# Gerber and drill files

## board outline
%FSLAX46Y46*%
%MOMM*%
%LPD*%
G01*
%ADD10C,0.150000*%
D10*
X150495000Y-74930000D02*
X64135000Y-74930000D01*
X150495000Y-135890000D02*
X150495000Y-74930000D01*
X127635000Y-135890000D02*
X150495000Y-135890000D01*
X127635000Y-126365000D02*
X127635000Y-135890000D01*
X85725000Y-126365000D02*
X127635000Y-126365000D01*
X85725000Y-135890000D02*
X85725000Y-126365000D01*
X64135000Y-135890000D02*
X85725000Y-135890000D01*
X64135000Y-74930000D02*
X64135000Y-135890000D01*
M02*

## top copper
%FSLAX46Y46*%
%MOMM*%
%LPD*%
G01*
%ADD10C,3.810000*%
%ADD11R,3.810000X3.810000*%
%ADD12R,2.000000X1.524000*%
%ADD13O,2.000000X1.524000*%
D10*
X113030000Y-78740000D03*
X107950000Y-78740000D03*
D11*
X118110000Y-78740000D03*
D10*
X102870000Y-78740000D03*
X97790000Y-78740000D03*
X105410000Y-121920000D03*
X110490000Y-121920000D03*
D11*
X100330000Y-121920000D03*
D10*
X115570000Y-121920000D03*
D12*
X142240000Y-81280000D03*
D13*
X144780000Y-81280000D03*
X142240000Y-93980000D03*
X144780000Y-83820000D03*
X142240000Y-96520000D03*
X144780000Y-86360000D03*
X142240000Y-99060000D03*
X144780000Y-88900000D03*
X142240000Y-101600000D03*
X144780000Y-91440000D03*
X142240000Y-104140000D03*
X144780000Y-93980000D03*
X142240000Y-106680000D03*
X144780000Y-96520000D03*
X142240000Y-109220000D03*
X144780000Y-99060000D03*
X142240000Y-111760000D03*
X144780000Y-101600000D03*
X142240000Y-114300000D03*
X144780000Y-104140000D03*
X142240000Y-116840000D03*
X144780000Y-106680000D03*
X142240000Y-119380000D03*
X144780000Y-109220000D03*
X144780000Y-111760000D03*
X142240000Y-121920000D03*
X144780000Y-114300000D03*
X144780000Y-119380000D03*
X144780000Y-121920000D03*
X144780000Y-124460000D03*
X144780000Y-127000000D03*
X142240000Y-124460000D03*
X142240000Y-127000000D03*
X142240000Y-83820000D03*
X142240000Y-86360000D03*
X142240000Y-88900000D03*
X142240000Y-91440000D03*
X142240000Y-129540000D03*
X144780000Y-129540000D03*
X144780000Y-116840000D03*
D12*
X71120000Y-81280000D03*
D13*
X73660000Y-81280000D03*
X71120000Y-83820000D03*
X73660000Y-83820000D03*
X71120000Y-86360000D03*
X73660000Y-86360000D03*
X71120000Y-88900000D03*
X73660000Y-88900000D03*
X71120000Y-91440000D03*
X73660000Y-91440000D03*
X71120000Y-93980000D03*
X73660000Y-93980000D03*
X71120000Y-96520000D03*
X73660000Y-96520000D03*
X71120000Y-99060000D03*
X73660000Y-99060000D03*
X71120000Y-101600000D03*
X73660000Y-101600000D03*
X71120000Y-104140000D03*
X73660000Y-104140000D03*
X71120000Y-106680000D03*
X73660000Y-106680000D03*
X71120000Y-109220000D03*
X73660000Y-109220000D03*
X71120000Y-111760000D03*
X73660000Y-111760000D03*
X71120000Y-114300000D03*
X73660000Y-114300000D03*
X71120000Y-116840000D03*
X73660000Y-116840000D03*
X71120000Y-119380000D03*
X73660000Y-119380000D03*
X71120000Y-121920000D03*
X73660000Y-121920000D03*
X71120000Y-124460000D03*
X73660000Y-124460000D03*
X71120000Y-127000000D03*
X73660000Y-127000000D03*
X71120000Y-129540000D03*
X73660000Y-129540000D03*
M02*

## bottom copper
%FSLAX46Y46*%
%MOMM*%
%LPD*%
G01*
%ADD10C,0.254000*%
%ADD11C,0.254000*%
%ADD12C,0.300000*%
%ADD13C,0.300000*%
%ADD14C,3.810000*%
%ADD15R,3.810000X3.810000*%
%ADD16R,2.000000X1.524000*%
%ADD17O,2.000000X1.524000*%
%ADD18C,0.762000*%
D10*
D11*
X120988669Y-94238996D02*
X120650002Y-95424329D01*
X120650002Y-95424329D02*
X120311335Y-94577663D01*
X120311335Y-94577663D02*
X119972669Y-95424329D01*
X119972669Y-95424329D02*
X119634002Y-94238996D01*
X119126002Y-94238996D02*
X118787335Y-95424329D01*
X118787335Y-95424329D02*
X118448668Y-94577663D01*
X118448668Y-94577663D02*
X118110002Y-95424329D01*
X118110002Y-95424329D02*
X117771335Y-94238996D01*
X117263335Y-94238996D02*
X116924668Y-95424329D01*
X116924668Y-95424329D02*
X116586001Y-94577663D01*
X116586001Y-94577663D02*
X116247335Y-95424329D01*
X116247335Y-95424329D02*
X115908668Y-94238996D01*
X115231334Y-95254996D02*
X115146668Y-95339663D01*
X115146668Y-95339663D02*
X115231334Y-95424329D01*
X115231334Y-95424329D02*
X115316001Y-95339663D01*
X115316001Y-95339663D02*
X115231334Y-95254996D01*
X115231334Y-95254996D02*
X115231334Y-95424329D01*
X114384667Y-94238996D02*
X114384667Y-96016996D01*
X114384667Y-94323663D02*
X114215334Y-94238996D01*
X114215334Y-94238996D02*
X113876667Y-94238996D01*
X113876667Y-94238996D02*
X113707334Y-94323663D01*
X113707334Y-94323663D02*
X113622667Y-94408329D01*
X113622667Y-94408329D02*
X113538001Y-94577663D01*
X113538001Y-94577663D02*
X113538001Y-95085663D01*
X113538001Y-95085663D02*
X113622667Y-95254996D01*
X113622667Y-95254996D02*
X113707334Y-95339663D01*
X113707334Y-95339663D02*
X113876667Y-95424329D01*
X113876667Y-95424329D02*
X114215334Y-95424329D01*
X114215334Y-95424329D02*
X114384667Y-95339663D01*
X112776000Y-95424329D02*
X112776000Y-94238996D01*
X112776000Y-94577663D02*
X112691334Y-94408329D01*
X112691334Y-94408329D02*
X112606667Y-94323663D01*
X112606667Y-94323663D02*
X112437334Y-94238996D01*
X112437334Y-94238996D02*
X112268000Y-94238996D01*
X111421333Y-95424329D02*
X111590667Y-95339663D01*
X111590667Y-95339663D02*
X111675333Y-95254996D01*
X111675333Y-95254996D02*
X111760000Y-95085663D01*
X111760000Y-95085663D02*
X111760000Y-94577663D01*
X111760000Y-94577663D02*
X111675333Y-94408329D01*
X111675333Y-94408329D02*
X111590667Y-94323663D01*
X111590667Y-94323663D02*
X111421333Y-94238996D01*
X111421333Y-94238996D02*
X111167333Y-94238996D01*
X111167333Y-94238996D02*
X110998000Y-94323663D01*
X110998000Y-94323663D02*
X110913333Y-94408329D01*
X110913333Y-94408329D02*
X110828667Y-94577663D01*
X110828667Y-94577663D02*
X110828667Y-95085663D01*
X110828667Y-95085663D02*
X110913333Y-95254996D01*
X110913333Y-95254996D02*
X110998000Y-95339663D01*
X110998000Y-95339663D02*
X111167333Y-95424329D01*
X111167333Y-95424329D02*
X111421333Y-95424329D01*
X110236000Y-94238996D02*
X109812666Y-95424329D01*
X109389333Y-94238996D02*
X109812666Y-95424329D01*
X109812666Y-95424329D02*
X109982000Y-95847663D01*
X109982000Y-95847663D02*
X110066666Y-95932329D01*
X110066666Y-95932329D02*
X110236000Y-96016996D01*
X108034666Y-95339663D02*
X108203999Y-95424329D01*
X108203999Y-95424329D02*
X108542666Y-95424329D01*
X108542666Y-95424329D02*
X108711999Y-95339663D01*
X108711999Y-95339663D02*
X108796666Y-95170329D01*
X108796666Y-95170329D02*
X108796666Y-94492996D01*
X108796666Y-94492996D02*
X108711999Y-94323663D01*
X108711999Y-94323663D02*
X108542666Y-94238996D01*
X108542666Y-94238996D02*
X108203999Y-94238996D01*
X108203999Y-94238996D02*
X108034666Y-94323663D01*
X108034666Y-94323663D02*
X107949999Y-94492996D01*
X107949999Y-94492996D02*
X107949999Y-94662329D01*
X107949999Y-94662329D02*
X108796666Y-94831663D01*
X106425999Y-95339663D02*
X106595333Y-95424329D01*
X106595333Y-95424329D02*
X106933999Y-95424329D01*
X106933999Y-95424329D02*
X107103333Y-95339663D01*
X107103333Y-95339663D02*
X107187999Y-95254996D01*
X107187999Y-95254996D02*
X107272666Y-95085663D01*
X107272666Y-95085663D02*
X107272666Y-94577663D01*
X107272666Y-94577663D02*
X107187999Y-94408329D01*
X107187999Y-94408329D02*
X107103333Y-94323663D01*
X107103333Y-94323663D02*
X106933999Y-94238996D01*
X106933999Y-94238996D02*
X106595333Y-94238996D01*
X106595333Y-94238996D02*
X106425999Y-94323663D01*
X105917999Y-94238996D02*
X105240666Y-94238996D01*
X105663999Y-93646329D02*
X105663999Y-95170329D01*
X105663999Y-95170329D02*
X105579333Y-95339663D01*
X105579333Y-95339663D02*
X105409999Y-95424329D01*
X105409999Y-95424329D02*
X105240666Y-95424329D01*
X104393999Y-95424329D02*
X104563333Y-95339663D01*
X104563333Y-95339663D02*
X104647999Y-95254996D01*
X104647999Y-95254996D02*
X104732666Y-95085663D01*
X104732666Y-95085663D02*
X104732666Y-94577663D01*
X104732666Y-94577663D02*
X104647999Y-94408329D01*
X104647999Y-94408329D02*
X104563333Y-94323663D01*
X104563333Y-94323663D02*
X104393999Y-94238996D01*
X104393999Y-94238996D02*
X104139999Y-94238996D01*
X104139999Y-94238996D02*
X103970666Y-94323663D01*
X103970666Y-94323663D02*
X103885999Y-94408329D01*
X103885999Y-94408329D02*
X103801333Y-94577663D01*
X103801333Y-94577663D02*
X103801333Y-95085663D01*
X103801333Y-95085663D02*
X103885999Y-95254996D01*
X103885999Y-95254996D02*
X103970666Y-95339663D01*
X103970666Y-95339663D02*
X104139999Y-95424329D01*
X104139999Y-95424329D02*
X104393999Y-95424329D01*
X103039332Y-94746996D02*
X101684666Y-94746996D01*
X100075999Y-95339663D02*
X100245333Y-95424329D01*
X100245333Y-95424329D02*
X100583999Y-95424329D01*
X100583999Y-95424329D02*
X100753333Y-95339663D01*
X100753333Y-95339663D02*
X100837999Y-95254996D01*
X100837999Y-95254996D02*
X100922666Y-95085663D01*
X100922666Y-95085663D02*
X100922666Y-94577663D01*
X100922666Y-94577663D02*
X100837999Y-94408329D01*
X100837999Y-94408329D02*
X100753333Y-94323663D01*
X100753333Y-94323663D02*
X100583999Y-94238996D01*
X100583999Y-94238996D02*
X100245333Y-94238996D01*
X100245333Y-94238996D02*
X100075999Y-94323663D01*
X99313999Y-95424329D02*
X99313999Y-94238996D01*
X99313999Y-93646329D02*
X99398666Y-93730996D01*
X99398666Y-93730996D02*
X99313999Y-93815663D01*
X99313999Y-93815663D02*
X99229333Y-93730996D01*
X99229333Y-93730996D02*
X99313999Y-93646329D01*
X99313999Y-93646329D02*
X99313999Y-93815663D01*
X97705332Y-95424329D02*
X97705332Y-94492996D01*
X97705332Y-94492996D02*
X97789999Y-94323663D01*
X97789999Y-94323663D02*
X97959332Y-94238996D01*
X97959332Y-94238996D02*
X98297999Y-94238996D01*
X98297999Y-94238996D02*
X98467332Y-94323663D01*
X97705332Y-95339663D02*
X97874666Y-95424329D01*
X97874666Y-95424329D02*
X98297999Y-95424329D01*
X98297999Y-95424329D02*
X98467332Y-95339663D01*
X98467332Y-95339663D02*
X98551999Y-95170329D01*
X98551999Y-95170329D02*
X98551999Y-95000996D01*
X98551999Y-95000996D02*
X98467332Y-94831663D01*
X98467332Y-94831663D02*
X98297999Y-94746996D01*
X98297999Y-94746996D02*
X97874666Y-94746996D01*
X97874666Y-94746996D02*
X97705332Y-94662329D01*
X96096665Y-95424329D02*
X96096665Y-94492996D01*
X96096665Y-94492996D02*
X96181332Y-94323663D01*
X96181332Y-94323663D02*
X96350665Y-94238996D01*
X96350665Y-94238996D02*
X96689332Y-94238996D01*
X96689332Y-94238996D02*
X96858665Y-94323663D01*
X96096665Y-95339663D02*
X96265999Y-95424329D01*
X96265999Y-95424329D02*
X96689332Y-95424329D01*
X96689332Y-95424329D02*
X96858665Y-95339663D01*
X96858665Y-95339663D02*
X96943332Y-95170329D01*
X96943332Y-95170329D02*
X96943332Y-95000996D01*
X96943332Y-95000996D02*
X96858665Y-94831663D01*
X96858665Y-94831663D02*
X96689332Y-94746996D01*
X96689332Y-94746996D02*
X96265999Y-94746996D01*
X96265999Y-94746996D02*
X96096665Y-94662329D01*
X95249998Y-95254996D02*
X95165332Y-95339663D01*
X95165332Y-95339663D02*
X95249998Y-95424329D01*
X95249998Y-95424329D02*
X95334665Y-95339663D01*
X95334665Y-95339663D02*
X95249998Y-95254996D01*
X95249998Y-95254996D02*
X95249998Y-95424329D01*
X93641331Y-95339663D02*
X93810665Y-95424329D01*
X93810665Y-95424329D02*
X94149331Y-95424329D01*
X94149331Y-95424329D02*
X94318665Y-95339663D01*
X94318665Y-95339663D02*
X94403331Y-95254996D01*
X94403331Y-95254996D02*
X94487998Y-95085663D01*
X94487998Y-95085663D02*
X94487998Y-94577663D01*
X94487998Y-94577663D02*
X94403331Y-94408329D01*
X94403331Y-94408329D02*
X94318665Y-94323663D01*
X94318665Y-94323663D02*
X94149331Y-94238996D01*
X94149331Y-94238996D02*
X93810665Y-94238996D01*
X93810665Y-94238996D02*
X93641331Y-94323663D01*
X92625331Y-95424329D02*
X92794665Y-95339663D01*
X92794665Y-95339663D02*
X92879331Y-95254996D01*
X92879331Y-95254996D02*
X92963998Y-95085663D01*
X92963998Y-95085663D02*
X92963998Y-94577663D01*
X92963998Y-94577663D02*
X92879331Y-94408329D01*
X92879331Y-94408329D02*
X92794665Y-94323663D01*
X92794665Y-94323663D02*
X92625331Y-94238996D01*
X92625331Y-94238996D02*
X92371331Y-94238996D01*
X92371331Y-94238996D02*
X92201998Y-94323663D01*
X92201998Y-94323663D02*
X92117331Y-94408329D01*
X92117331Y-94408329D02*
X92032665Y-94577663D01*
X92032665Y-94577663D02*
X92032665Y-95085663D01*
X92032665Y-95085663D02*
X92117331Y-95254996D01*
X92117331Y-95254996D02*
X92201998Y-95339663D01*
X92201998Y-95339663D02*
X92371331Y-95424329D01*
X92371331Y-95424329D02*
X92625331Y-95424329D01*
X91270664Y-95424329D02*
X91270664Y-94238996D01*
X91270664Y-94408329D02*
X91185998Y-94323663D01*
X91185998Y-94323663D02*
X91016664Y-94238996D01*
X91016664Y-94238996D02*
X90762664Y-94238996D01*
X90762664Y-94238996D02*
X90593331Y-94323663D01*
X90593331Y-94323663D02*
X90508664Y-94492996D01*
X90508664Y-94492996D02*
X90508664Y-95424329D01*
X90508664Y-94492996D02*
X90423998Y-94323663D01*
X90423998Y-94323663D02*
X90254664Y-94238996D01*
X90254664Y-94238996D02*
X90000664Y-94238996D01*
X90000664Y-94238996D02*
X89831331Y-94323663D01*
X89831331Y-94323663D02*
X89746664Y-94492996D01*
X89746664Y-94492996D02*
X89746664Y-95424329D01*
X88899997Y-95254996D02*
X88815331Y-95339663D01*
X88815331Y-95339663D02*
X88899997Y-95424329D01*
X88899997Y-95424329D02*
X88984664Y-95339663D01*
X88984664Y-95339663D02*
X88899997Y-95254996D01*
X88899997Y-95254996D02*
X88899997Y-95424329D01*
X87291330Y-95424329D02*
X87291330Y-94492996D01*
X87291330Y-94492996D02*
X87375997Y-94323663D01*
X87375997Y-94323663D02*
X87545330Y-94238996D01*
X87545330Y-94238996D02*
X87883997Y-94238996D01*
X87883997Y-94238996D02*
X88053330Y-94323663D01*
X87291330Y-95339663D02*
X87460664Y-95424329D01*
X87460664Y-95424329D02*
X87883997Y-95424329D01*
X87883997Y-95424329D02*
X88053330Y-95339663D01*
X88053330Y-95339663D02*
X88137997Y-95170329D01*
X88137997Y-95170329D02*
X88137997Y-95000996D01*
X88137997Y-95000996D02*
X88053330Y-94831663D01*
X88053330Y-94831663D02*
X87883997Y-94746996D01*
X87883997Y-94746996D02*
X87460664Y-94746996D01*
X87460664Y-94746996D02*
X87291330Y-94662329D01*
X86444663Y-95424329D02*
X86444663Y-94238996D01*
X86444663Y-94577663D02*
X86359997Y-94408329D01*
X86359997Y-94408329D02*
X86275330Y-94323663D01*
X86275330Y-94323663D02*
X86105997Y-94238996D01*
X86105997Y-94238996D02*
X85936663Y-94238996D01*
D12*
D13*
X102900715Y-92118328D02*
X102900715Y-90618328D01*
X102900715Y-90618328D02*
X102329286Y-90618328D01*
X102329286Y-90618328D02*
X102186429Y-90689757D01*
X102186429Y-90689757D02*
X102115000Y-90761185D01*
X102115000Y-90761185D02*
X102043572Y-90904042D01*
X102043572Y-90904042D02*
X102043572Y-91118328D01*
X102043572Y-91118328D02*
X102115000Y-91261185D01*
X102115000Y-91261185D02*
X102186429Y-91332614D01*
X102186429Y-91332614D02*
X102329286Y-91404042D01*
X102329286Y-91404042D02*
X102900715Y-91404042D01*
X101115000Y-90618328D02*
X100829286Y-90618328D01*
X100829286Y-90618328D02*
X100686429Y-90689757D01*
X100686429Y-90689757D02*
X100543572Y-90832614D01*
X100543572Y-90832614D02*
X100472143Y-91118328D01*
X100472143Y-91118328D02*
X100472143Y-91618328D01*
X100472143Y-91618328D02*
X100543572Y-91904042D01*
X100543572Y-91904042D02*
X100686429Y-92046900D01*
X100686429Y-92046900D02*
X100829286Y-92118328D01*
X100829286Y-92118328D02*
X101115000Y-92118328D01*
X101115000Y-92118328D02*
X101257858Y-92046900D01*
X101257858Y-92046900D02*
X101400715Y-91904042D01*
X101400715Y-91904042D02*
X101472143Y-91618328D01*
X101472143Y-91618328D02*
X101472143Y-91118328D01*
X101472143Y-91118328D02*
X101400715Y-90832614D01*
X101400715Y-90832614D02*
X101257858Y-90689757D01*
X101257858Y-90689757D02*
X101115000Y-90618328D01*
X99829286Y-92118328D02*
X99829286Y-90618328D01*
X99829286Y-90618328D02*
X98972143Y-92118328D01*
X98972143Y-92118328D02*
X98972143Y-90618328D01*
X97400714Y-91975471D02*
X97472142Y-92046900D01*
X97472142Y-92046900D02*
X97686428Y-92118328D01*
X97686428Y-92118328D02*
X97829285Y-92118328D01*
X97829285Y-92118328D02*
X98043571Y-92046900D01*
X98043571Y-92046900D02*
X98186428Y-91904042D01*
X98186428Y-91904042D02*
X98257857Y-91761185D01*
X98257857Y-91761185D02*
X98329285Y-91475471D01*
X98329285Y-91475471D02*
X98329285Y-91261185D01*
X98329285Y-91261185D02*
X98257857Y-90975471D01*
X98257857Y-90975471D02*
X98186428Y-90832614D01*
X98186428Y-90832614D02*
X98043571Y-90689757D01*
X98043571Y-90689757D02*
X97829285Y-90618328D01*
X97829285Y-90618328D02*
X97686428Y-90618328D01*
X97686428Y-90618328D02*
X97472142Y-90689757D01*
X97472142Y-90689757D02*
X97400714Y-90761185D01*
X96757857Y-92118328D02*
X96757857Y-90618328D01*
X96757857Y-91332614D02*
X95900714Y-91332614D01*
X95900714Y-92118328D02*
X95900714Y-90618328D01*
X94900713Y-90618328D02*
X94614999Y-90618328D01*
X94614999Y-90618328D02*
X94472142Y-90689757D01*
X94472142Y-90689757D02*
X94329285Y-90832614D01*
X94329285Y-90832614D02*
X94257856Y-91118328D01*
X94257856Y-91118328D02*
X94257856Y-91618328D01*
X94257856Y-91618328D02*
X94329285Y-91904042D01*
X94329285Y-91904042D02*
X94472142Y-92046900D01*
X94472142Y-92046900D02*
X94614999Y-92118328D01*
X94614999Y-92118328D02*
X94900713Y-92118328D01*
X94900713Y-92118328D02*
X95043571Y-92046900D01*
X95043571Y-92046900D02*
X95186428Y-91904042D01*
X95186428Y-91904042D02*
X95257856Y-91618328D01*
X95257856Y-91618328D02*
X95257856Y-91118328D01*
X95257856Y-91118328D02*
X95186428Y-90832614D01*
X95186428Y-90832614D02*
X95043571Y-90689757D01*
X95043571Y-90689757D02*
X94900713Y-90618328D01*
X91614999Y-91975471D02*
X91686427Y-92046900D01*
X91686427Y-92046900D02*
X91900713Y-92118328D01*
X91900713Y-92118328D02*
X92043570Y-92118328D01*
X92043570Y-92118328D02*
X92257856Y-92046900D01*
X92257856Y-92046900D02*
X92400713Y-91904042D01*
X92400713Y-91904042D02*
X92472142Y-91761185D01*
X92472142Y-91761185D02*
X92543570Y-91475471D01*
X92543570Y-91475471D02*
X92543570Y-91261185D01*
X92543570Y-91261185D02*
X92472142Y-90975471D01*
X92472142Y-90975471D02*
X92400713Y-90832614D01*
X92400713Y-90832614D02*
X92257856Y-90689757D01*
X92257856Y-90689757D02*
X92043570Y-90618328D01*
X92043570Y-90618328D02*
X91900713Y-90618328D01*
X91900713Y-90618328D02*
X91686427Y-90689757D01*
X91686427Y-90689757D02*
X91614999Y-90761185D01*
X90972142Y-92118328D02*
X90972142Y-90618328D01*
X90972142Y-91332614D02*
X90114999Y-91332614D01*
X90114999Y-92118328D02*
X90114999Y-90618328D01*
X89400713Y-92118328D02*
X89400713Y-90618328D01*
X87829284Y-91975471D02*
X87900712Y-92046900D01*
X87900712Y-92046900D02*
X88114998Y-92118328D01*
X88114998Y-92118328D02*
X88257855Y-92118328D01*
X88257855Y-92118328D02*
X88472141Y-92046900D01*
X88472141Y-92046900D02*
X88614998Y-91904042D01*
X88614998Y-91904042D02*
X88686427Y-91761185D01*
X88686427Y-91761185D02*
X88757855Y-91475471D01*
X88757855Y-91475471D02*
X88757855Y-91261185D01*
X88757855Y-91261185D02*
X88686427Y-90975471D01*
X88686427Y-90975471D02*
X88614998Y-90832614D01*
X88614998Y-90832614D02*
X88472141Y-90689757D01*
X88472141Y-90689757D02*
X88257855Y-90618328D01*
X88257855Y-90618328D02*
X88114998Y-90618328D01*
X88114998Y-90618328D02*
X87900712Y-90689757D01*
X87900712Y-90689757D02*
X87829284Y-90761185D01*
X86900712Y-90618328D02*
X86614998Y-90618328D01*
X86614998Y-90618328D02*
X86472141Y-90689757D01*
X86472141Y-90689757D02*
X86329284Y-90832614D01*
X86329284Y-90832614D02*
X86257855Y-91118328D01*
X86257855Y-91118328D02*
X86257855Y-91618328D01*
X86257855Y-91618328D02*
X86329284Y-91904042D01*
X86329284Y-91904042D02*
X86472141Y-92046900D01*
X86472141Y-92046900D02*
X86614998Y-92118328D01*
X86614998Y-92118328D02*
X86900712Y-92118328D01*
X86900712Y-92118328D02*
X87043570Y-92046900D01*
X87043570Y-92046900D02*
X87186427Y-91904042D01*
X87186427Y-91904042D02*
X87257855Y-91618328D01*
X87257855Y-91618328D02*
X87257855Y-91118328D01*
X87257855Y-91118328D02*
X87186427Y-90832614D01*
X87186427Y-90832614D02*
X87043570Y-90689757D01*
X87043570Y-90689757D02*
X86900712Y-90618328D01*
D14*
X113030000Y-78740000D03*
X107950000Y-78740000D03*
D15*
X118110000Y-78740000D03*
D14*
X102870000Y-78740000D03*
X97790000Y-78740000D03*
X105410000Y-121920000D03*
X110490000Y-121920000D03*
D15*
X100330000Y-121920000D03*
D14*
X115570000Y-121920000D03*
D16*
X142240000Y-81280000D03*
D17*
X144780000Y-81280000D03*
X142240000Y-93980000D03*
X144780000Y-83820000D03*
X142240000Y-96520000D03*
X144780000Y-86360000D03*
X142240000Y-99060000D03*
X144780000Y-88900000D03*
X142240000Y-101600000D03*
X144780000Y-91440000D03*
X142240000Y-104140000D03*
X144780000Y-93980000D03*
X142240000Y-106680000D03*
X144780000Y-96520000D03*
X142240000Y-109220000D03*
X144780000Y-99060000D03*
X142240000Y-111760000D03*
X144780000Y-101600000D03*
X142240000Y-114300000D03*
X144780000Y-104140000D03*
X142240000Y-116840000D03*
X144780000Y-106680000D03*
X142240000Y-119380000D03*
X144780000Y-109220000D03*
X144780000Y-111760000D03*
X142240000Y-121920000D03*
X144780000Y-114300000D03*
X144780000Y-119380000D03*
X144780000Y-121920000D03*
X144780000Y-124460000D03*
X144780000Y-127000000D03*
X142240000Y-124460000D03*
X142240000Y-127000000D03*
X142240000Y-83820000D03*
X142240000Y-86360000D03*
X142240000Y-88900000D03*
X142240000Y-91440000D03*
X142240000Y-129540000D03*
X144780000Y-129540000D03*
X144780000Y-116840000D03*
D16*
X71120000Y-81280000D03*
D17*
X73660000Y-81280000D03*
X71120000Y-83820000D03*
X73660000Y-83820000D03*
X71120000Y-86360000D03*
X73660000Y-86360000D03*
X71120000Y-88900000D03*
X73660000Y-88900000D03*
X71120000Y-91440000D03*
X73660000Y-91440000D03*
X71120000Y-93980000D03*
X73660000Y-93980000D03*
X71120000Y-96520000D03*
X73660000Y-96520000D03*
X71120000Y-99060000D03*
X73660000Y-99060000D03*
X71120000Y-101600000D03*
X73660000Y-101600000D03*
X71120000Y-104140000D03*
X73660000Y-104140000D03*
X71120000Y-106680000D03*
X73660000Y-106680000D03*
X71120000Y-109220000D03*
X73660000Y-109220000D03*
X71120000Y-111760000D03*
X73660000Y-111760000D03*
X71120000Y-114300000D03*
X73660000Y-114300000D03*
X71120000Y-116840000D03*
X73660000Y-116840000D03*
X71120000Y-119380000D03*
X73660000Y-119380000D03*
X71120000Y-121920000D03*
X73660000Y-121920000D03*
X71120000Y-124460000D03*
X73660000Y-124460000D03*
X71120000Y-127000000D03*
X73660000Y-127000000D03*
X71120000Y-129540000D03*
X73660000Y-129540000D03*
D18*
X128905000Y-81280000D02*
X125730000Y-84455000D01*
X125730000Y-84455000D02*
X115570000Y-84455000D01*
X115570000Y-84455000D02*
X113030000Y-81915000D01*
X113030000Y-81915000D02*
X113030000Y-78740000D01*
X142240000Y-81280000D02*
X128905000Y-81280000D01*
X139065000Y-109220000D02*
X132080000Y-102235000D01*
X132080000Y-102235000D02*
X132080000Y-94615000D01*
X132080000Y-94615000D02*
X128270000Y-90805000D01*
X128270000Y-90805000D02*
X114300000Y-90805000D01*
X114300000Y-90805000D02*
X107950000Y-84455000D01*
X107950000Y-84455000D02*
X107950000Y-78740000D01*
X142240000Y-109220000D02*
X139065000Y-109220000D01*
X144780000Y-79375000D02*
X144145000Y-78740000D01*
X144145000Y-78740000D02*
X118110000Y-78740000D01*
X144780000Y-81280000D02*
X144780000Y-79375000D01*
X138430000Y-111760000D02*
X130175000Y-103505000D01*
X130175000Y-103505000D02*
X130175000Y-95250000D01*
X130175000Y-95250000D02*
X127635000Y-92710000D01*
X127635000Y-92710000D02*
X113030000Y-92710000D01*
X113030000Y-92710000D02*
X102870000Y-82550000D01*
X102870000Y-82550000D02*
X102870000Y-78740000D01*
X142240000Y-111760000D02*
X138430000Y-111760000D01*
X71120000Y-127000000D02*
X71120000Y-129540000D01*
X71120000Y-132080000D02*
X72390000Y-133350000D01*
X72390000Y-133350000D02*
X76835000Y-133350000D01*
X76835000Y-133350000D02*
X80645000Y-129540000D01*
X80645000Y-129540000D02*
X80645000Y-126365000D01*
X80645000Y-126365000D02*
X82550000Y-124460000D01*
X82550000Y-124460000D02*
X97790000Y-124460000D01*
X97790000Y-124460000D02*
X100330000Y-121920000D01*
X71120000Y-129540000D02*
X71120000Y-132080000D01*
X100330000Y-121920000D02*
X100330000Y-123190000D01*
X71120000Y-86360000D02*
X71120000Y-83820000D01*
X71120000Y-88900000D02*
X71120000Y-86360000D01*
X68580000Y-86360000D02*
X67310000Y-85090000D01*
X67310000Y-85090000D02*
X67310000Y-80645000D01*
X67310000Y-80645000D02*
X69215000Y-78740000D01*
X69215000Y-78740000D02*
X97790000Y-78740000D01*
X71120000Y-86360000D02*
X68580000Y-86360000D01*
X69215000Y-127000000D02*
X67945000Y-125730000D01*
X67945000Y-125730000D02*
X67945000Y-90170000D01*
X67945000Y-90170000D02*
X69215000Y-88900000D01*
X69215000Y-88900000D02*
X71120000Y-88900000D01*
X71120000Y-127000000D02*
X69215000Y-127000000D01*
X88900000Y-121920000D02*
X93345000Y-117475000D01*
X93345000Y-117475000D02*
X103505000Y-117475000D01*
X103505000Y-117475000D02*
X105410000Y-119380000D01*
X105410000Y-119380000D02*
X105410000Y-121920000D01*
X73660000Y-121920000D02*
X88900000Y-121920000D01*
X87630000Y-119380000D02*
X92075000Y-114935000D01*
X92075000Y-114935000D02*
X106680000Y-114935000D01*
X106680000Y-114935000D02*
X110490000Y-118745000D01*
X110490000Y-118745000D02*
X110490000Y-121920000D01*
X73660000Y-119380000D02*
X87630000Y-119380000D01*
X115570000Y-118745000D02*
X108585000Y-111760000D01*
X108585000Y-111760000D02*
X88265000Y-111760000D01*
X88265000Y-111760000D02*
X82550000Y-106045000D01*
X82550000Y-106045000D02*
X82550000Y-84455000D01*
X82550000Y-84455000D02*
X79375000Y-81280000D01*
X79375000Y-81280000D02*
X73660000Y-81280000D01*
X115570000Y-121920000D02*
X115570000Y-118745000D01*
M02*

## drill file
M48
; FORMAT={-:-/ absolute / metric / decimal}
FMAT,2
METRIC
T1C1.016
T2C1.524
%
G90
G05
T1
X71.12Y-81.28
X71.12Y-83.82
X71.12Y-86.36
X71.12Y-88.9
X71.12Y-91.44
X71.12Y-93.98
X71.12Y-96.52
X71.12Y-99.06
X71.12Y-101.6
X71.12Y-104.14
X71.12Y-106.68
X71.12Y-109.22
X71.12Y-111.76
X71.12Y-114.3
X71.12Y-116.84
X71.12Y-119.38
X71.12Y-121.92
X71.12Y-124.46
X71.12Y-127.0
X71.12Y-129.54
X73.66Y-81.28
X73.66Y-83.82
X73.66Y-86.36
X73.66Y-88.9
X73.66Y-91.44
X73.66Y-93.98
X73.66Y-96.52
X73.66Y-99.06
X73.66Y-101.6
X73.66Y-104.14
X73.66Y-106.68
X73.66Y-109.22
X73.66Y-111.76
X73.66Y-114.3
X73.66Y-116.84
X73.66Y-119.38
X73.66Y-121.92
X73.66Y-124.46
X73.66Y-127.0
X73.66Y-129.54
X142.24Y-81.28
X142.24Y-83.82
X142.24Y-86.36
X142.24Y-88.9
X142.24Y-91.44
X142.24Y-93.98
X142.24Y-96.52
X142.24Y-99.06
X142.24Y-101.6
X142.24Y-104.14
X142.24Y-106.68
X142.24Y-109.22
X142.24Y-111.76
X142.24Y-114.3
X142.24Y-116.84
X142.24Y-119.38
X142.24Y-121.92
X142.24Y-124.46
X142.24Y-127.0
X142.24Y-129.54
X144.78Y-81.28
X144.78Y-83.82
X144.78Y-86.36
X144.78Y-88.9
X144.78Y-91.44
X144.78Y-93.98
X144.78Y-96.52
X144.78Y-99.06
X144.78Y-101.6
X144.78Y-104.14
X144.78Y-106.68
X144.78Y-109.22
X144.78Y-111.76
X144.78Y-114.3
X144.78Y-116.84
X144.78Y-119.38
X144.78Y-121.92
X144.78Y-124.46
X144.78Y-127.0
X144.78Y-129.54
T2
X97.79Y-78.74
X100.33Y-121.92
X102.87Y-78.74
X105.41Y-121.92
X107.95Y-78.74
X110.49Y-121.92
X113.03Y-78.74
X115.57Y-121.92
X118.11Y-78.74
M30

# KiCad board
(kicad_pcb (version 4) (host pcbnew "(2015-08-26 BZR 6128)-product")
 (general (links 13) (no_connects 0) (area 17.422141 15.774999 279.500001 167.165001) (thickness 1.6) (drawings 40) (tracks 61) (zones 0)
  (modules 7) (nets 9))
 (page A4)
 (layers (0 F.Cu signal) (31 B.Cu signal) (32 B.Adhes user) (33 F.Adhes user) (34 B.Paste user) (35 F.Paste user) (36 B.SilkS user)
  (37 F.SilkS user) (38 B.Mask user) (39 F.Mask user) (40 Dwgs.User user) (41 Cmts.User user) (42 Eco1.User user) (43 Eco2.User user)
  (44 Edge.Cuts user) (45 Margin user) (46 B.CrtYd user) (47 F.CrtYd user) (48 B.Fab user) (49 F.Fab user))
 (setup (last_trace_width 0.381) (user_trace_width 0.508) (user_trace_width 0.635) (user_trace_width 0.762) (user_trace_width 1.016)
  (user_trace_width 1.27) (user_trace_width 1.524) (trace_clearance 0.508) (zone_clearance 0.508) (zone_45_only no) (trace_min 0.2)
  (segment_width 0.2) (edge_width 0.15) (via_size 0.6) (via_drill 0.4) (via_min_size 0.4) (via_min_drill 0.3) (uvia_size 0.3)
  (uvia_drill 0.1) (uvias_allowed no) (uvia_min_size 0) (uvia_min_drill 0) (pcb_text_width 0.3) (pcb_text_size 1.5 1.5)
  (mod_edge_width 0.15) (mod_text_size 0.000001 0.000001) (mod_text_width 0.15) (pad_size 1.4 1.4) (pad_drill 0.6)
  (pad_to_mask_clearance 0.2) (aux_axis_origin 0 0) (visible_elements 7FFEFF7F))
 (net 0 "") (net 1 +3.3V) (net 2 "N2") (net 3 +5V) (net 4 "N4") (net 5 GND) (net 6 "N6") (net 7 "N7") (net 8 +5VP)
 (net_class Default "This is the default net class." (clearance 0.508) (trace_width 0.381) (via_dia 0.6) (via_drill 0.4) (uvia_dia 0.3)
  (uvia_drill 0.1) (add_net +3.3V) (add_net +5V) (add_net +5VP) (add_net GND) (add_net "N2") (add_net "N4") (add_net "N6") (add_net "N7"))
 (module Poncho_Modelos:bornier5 (layer F.Cu) (at 107.95 78.74 180)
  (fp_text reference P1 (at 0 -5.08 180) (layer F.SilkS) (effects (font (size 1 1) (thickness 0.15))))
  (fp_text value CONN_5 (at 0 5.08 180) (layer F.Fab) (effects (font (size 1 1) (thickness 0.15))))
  (pad 2 thru_hole circle (at -5.08 0 180) (size 3.81 3.81) (drill 1.524) (layers *.Cu *.Mask F.SilkS) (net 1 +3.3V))
  (pad 3 thru_hole circle (at 0 0 180) (size 3.81 3.81) (drill 1.524) (layers *.Cu *.Mask F.SilkS) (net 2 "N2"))
  (pad 1 thru_hole rect (at -10.16 0 180) (size 3.81 3.81) (drill 1.524) (layers *.Cu *.Mask F.SilkS) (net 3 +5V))
  (pad 4 thru_hole circle (at 5.08 0 180) (size 3.81 3.81) (drill 1.524) (layers *.Cu *.Mask F.SilkS) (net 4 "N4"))
  (pad 5 thru_hole circle (at 10.16 0 180) (size 3.81 3.81) (drill 1.524) (layers *.Cu *.Mask F.SilkS) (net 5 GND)))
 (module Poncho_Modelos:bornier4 (layer F.Cu) (at 107.95 121.92)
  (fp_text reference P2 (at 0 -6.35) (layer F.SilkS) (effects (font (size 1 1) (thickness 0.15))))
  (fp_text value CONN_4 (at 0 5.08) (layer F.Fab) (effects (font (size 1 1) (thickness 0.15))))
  (pad 2 thru_hole circle (at -2.54 0) (size 3.81 3.81) (drill 1.524) (layers *.Cu *.Mask F.SilkS) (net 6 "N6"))
  (pad 3 thru_hole circle (at 2.54 0) (size 3.81 3.81) (drill 1.524) (layers *.Cu *.Mask F.SilkS) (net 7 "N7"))
  (pad 1 thru_hole rect (at -7.62 0) (size 3.81 3.81) (drill 1.524) (layers *.Cu *.Mask F.SilkS) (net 5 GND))
  (pad 4 thru_hole circle (at 7.62 0) (size 3.81 3.81) (drill 1.524) (layers *.Cu *.Mask F.SilkS) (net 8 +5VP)))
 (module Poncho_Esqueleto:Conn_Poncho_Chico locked (layer F.Cu) (at 142.24 81.28)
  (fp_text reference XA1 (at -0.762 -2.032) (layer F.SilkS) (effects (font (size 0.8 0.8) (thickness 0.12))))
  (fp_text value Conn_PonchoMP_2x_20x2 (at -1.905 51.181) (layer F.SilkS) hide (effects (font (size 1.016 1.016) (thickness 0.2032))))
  (pad 1 thru_hole rect (at 0 0 270) (size 1.524 2) (drill 1.016) (layers *.Cu *.Mask F.SilkS) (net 1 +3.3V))
  (pad 2 thru_hole oval (at 2.54 0 270) (size 1.524 2) (drill 1.016) (layers *.Cu *.Mask F.SilkS) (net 3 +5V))
  (pad 11 thru_hole oval (at 0 12.7 270) (size 1.524 2) (drill 1.016) (layers *.Cu *.Mask F.SilkS))
  (pad 4 thru_hole oval (at 2.54 2.54 270) (size 1.524 2) (drill 1.016) (layers *.Cu *.Mask F.SilkS))
  (pad 13 thru_hole oval (at 0 15.24 270) (size 1.524 2) (drill 1.016) (layers *.Cu *.Mask F.SilkS))
  (pad 6 thru_hole oval (at 2.54 5.08 270) (size 1.524 2) (drill 1.016) (layers *.Cu *.Mask F.SilkS))
  (pad 15 thru_hole oval (at 0 17.78 270) (size 1.524 2) (drill 1.016) (layers *.Cu *.Mask F.SilkS))
  (pad 8 thru_hole oval (at 2.54 7.62 270) (size 1.524 2) (drill 1.016) (layers *.Cu *.Mask F.SilkS))
  (pad 17 thru_hole oval (at 0 20.32 270) (size 1.524 2) (drill 1.016) (layers *.Cu *.Mask F.SilkS))
  (pad 10 thru_hole oval (at 2.54 10.16 270) (size 1.524 2) (drill 1.016) (layers *.Cu *.Mask F.SilkS))
  (pad 19 thru_hole oval (at 0 22.86 270) (size 1.524 2) (drill 1.016) (layers *.Cu *.Mask F.SilkS))
  (pad 12 thru_hole oval (at 2.54 12.7 270) (size 1.524 2) (drill 1.016) (layers *.Cu *.Mask F.SilkS))
  (pad 21 thru_hole oval (at 0 25.4 270) (size 1.524 2) (drill 1.016) (layers *.Cu *.Mask F.SilkS))
  (pad 14 thru_hole oval (at 2.54 15.24 270) (size 1.524 2) (drill 1.016) (layers *.Cu *.Mask F.SilkS))
  (pad 23 thru_hole oval (at 0 27.94 270) (size 1.524 2) (drill 1.016) (layers *.Cu *.Mask F.SilkS) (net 2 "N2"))
  (pad 16 thru_hole oval (at 2.54 17.78 270) (size 1.524 2) (drill 1.016) (layers *.Cu *.Mask F.SilkS))
  (pad 25 thru_hole oval (at 0 30.48 270) (size 1.524 2) (drill 1.016) (layers *.Cu *.Mask F.SilkS) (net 4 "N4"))
  (pad 18 thru_hole oval (at 2.54 20.32 270) (size 1.524 2) (drill 1.016) (layers *.Cu *.Mask F.SilkS))
  (pad 27 thru_hole oval (at 0 33.02 270) (size 1.524 2) (drill 1.016) (layers *.Cu *.Mask F.SilkS))
  (pad 20 thru_hole oval (at 2.54 22.86 270) (size 1.524 2) (drill 1.016) (layers *.Cu *.Mask F.SilkS))
  (pad 29 thru_hole oval (at 0 35.56 270) (size 1.524 2) (drill 1.016) (layers *.Cu *.Mask F.SilkS))
  (pad 22 thru_hole oval (at 2.54 25.4 270) (size 1.524 2) (drill 1.016) (layers *.Cu *.Mask F.SilkS))
  (pad 31 thru_hole oval (at 0 38.1 270) (size 1.524 2) (drill 1.016) (layers *.Cu *.Mask F.SilkS))
  (pad 24 thru_hole oval (at 2.54 27.94 270) (size 1.524 2) (drill 1.016) (layers *.Cu *.Mask F.SilkS))
  (pad 26 thru_hole oval (at 2.54 30.48 270) (size 1.524 2) (drill 1.016) (layers *.Cu *.Mask F.SilkS))
  (pad 33 thru_hole oval (at 0 40.64 270) (size 1.524 2) (drill 1.016) (layers *.Cu *.Mask F.SilkS))
  (pad 28 thru_hole oval (at 2.54 33.02 270) (size 1.524 2) (drill 1.016) (layers *.Cu *.Mask F.SilkS))
  (pad 32 thru_hole oval (at 2.54 38.1 270) (size 1.524 2) (drill 1.016) (layers *.Cu *.Mask F.SilkS))
  (pad 34 thru_hole oval (at 2.54 40.64 270) (size 1.524 2) (drill 1.016) (layers *.Cu *.Mask F.SilkS))
  (pad 36 thru_hole oval (at 2.54 43.18 270) (size 1.524 2) (drill 1.016) (layers *.Cu *.Mask F.SilkS))
  (pad 38 thru_hole oval (at 2.54 45.72 270) (size 1.524 2) (drill 1.016) (layers *.Cu *.Mask F.SilkS))
  (pad 35 thru_hole oval (at 0 43.18 270) (size 1.524 2) (drill 1.016) (layers *.Cu *.Mask F.SilkS))
  (pad 37 thru_hole oval (at 0 45.72 270) (size 1.524 2) (drill 1.016) (layers *.Cu *.Mask F.SilkS))
  (pad 3 thru_hole oval (at 0 2.54 270) (size 1.524 2) (drill 1.016) (layers *.Cu *.Mask F.SilkS))
  (pad 5 thru_hole oval (at 0 5.08 270) (size 1.524 2) (drill 1.016) (layers *.Cu *.Mask F.SilkS))
  (pad 7 thru_hole oval (at 0 7.62 270) (size 1.524 2) (drill 1.016) (layers *.Cu *.Mask F.SilkS))
  (pad 9 thru_hole oval (at 0 10.16 270) (size 1.524 2) (drill 1.016) (layers *.Cu *.Mask F.SilkS))
  (pad 39 thru_hole oval (at 0 48.26 270) (size 1.524 2) (drill 1.016) (layers *.Cu *.Mask F.SilkS))
  (pad 40 thru_hole oval (at 2.54 48.26 270) (size 1.524 2) (drill 1.016) (layers *.Cu *.Mask F.SilkS))
  (pad 30 thru_hole oval (at 2.54 35.56 270) (size 1.524 2) (drill 1.016) (layers *.Cu *.Mask F.SilkS))
  (pad 41 thru_hole rect (at -71.12 0 270) (size 1.524 2) (drill 1.016) (layers *.Cu *.Mask F.SilkS))
  (pad 42 thru_hole oval (at -68.58 0 270) (size 1.524 2) (drill 1.016) (layers *.Cu *.Mask F.SilkS) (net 8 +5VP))
  (pad 43 thru_hole oval (at -71.12 2.54 270) (size 1.524 2) (drill 1.016) (layers *.Cu *.Mask F.SilkS) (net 5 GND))
  (pad 44 thru_hole oval (at -68.58 2.54 270) (size 1.524 2) (drill 1.016) (layers *.Cu *.Mask F.SilkS))
  (pad 45 thru_hole oval (at -71.12 5.08 270) (size 1.524 2) (drill 1.016) (layers *.Cu *.Mask F.SilkS) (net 5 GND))
  (pad 46 thru_hole oval (at -68.58 5.08 270) (size 1.524 2) (drill 1.016) (layers *.Cu *.Mask F.SilkS))
  (pad 47 thru_hole oval (at -71.12 7.62 270) (size 1.524 2) (drill 1.016) (layers *.Cu *.Mask F.SilkS) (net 5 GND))
  (pad 48 thru_hole oval (at -68.58 7.62 270) (size 1.524 2) (drill 1.016) (layers *.Cu *.Mask F.SilkS))
  (pad 49 thru_hole oval (at -71.12 10.16 270) (size 1.524 2) (drill 1.016) (layers *.Cu *.Mask F.SilkS))
  (pad 50 thru_hole oval (at -68.58 10.16 270) (size 1.524 2) (drill 1.016) (layers *.Cu *.Mask F.SilkS))
  (pad 51 thru_hole oval (at -71.12 12.7 270) (size 1.524 2) (drill 1.016) (layers *.Cu *.Mask F.SilkS))
  (pad 52 thru_hole oval (at -68.58 12.7 270) (size 1.524 2) (drill 1.016) (layers *.Cu *.Mask F.SilkS))
  (pad 53 thru_hole oval (at -71.12 15.24 270) (size 1.524 2) (drill 1.016) (layers *.Cu *.Mask F.SilkS))
  (pad 54 thru_hole oval (at -68.58 15.24 270) (size 1.524 2) (drill 1.016) (layers *.Cu *.Mask F.SilkS))
  (pad 55 thru_hole oval (at -71.12 17.78 270) (size 1.524 2) (drill 1.016) (layers *.Cu *.Mask F.SilkS))
  (pad 56 thru_hole oval (at -68.58 17.78 270) (size 1.524 2) (drill 1.016) (layers *.Cu *.Mask F.SilkS))
  (pad 57 thru_hole oval (at -71.12 20.32 270) (size 1.524 2) (drill 1.016) (layers *.Cu *.Mask F.SilkS))
  (pad 58 thru_hole oval (at -68.58 20.32 270) (size 1.524 2) (drill 1.016) (layers *.Cu *.Mask F.SilkS))
  (pad 59 thru_hole oval (at -71.12 22.86 270) (size 1.524 2) (drill 1.016) (layers *.Cu *.Mask F.SilkS))
  (pad 60 thru_hole oval (at -68.58 22.86 270) (size 1.524 2) (drill 1.016) (layers *.Cu *.Mask F.SilkS))
  (pad 61 thru_hole oval (at -71.12 25.4 270) (size 1.524 2) (drill 1.016) (layers *.Cu *.Mask F.SilkS))
  (pad 62 thru_hole oval (at -68.58 25.4 270) (size 1.524 2) (drill 1.016) (layers *.Cu *.Mask F.SilkS))
  (pad 63 thru_hole oval (at -71.12 27.94 270) (size 1.524 2) (drill 1.016) (layers *.Cu *.Mask F.SilkS))
  (pad 64 thru_hole oval (at -68.58 27.94 270) (size 1.524 2) (drill 1.016) (layers *.Cu *.Mask F.SilkS))
  (pad 65 thru_hole oval (at -71.12 30.48 270) (size 1.524 2) (drill 1.016) (layers *.Cu *.Mask F.SilkS))
  (pad 66 thru_hole oval (at -68.58 30.48 270) (size 1.524 2) (drill 1.016) (layers *.Cu *.Mask F.SilkS))
  (pad 67 thru_hole oval (at -71.12 33.02 270) (size 1.524 2) (drill 1.016) (layers *.Cu *.Mask F.SilkS))
  (pad 68 thru_hole oval (at -68.58 33.02 270) (size 1.524 2) (drill 1.016) (layers *.Cu *.Mask F.SilkS))
  (pad 69 thru_hole oval (at -71.12 35.56 270) (size 1.524 2) (drill 1.016) (layers *.Cu *.Mask F.SilkS))
  (pad 70 thru_hole oval (at -68.58 35.56 270) (size 1.524 2) (drill 1.016) (layers *.Cu *.Mask F.SilkS))
  (pad 71 thru_hole oval (at -71.12 38.1 270) (size 1.524 2) (drill 1.016) (layers *.Cu *.Mask F.SilkS))
  (pad 72 thru_hole oval (at -68.58 38.1 270) (size 1.524 2) (drill 1.016) (layers *.Cu *.Mask F.SilkS) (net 7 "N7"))
  (pad 73 thru_hole oval (at -71.12 40.64 270) (size 1.524 2) (drill 1.016) (layers *.Cu *.Mask F.SilkS))
  (pad 74 thru_hole oval (at -68.58 40.64 270) (size 1.524 2) (drill 1.016) (layers *.Cu *.Mask F.SilkS) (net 6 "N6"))
  (pad 75 thru_hole oval (at -71.12 43.18 270) (size 1.524 2) (drill 1.016) (layers *.Cu *.Mask F.SilkS))
  (pad 76 thru_hole oval (at -68.58 43.18 270) (size 1.524 2) (drill 1.016) (layers *.Cu *.Mask F.SilkS))
  (pad 77 thru_hole oval (at -71.12 45.72 270) (size 1.524 2) (drill 1.016) (layers *.Cu *.Mask F.SilkS) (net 5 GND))
  (pad 78 thru_hole oval (at -68.58 45.72 270) (size 1.524 2) (drill 1.016) (layers *.Cu *.Mask F.SilkS))
  (pad 79 thru_hole oval (at -71.12 48.26 270) (size 1.524 2) (drill 1.016) (layers *.Cu *.Mask F.SilkS) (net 5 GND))
  (pad 80 thru_hole oval (at -68.58 48.26 270) (size 1.524 2) (drill 1.016) (layers *.Cu *.Mask F.SilkS)))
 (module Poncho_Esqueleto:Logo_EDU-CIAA (layer F.Cu) (at 114.3 100.965)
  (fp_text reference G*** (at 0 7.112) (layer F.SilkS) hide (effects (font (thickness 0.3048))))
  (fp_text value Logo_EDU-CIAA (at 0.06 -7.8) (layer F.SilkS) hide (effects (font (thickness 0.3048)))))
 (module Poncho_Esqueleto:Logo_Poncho (layer F.Cu) (at 90.805 100.965)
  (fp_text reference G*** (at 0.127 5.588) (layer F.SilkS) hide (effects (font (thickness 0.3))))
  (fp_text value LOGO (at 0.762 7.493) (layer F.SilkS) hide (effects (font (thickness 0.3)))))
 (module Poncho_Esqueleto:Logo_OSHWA (layer F.Cu) (at 101.6 100.965)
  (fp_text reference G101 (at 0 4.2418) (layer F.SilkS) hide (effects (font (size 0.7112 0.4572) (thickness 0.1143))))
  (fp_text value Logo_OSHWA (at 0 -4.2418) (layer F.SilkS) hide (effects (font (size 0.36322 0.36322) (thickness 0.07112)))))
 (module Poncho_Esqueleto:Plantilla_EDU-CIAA (layer F.Cu) (at 142.24 81.28)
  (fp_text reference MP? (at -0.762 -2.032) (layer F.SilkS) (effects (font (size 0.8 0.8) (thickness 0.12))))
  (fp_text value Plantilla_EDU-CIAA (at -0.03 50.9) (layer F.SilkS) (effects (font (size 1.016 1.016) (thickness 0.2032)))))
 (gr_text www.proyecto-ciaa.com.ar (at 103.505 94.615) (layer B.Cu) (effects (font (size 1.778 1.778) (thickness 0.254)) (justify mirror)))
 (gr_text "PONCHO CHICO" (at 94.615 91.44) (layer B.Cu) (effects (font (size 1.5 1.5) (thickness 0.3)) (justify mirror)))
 (gr_line (start 150.495 74.93) (end 64.135 74.93) (angle 90) (layer Edge.Cuts) (width 0.15))
 (gr_line (start 150.495 135.89) (end 150.495 74.93) (angle 90) (layer Edge.Cuts) (width 0.15))
 (gr_line (start 127.635 135.89) (end 150.495 135.89) (angle 90) (layer Edge.Cuts) (width 0.15))
 (gr_line (start 127.635 126.365) (end 127.635 135.89) (angle 90) (layer Edge.Cuts) (width 0.15))
 (gr_line (start 85.725 126.365) (end 127.635 126.365) (angle 90) (layer Edge.Cuts) (width 0.15))
 (gr_line (start 85.725 135.89) (end 85.725 126.365) (angle 90) (layer Edge.Cuts) (width 0.15))
 (gr_line (start 64.135 135.89) (end 85.725 135.89) (angle 90) (layer Edge.Cuts) (width 0.15))
 (gr_line (start 64.135 74.93) (end 64.135 135.89) (angle 90) (layer Edge.Cuts) (width 0.15))
 (segment (start 128.905 81.28) (end 125.73 84.455) (width 0.762) (layer B.Cu) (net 1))
 (segment (start 125.73 84.455) (end 115.57 84.455) (width 0.762) (layer B.Cu) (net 1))
 (segment (start 115.57 84.455) (end 113.03 81.915) (width 0.762) (layer B.Cu) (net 1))
 (segment (start 113.03 81.915) (end 113.03 78.74) (width 0.762) (layer B.Cu) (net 1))
 (segment (start 142.24 81.28) (end 128.905 81.28) (width 0.762) (layer B.Cu) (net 1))
 (segment (start 139.065 109.22) (end 132.08 102.235) (width 0.762) (layer B.Cu) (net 2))
 (segment (start 132.08 102.235) (end 132.08 94.615) (width 0.762) (layer B.Cu) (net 2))
 (segment (start 132.08 94.615) (end 128.27 90.805) (width 0.762) (layer B.Cu) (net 2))
 (segment (start 128.27 90.805) (end 114.3 90.805) (width 0.762) (layer B.Cu) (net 2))
 (segment (start 114.3 90.805) (end 107.95 84.455) (width 0.762) (layer B.Cu) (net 2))
 (segment (start 107.95 84.455) (end 107.95 78.74) (width 0.762) (layer B.Cu) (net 2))
 (segment (start 142.24 109.22) (end 139.065 109.22) (width 0.762) (layer B.Cu) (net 2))
 (segment (start 144.78 79.375) (end 144.145 78.74) (width 0.762) (layer B.Cu) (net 3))
 (segment (start 144.145 78.74) (end 118.11 78.74) (width 0.762) (layer B.Cu) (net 3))
 (segment (start 144.78 81.28) (end 144.78 79.375) (width 0.762) (layer B.Cu) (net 3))
 (segment (start 138.43 111.76) (end 130.175 103.505) (width 0.762) (layer B.Cu) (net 4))
 (segment (start 130.175 103.505) (end 130.175 95.25) (width 0.762) (layer B.Cu) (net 4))
 (segment (start 130.175 95.25) (end 127.635 92.71) (width 0.762) (layer B.Cu) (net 4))
 (segment (start 127.635 92.71) (end 113.03 92.71) (width 0.762) (layer B.Cu) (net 4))
 (segment (start 113.03 92.71) (end 102.87 82.55) (width 0.762) (layer B.Cu) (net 4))
 (segment (start 102.87 82.55) (end 102.87 78.74) (width 0.762) (layer B.Cu) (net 4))
 (segment (start 142.24 111.76) (end 138.43 111.76) (width 0.762) (layer B.Cu) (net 4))
 (segment (start 71.12 127) (end 71.12 129.54) (width 0.762) (layer B.Cu) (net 5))
 (segment (start 71.12 132.08) (end 72.39 133.35) (width 0.762) (layer B.Cu) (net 5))
 (segment (start 72.39 133.35) (end 76.835 133.35) (width 0.762) (layer B.Cu) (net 5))
 (segment (start 76.835 133.35) (end 80.645 129.54) (width 0.762) (layer B.Cu) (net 5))
 (segment (start 80.645 129.54) (end 80.645 126.365) (width 0.762) (layer B.Cu) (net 5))
 (segment (start 80.645 126.365) (end 82.55 124.46) (width 0.762) (layer B.Cu) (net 5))
 (segment (start 82.55 124.46) (end 97.79 124.46) (width 0.762) (layer B.Cu) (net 5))
 (segment (start 97.79 124.46) (end 100.33 121.92) (width 0.762) (layer B.Cu) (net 5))
 (segment (start 71.12 129.54) (end 71.12 132.08) (width 0.762) (layer B.Cu) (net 5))
 (segment (start 100.33 121.92) (end 100.33 123.19) (width 0.762) (layer B.Cu) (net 5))
 (segment (start 71.12 86.36) (end 71.12 83.82) (width 0.762) (layer B.Cu) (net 5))
 (segment (start 71.12 88.9) (end 71.12 86.36) (width 0.762) (layer B.Cu) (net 5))
 (segment (start 68.58 86.36) (end 67.31 85.09) (width 0.762) (layer B.Cu) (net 5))
 (segment (start 67.31 85.09) (end 67.31 80.645) (width 0.762) (layer B.Cu) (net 5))
 (segment (start 67.31 80.645) (end 69.215 78.74) (width 0.762) (layer B.Cu) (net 5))
 (segment (start 69.215 78.74) (end 97.79 78.74) (width 0.762) (layer B.Cu) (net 5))
 (segment (start 71.12 86.36) (end 68.58 86.36) (width 0.762) (layer B.Cu) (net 5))
 (segment (start 69.215 127) (end 67.945 125.73) (width 0.762) (layer B.Cu) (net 5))
 (segment (start 67.945 125.73) (end 67.945 90.17) (width 0.762) (layer B.Cu) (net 5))
 (segment (start 67.945 90.17) (end 69.215 88.9) (width 0.762) (layer B.Cu) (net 5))
 (segment (start 69.215 88.9) (end 71.12 88.9) (width 0.762) (layer B.Cu) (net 5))
 (segment (start 71.12 127) (end 69.215 127) (width 0.762) (layer B.Cu) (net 5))
 (segment (start 88.9 121.92) (end 93.345 117.475) (width 0.762) (layer B.Cu) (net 6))
 (segment (start 93.345 117.475) (end 103.505 117.475) (width 0.762) (layer B.Cu) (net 6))
 (segment (start 103.505 117.475) (end 105.41 119.38) (width 0.762) (layer B.Cu) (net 6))
 (segment (start 105.41 119.38) (end 105.41 121.92) (width 0.762) (layer B.Cu) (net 6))
 (segment (start 73.66 121.92) (end 88.9 121.92) (width 0.762) (layer B.Cu) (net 6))
 (segment (start 87.63 119.38) (end 92.075 114.935) (width 0.762) (layer B.Cu) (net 7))
 (segment (start 92.075 114.935) (end 106.68 114.935) (width 0.762) (layer B.Cu) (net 7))
 (segment (start 106.68 114.935) (end 110.49 118.745) (width 0.762) (layer B.Cu) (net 7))
 (segment (start 110.49 118.745) (end 110.49 121.92) (width 0.762) (layer B.Cu) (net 7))
 (segment (start 73.66 119.38) (end 87.63 119.38) (width 0.762) (layer B.Cu) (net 7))
 (segment (start 115.57 118.745) (end 108.585 111.76) (width 0.762) (layer B.Cu) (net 8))
 (segment (start 108.585 111.76) (end 88.265 111.76) (width 0.762) (layer B.Cu) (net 8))
 (segment (start 88.265 111.76) (end 82.55 106.045) (width 0.762) (layer B.Cu) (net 8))
 (segment (start 82.55 106.045) (end 82.55 84.455) (width 0.762) (layer B.Cu) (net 8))
 (segment (start 82.55 84.455) (end 79.375 81.28) (width 0.762) (layer B.Cu) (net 8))
 (segment (start 79.375 81.28) (end 73.66 81.28) (width 0.762) (layer B.Cu) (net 8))
 (segment (start 115.57 121.92) (end 115.57 118.745) (width 0.762) (layer B.Cu) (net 8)))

